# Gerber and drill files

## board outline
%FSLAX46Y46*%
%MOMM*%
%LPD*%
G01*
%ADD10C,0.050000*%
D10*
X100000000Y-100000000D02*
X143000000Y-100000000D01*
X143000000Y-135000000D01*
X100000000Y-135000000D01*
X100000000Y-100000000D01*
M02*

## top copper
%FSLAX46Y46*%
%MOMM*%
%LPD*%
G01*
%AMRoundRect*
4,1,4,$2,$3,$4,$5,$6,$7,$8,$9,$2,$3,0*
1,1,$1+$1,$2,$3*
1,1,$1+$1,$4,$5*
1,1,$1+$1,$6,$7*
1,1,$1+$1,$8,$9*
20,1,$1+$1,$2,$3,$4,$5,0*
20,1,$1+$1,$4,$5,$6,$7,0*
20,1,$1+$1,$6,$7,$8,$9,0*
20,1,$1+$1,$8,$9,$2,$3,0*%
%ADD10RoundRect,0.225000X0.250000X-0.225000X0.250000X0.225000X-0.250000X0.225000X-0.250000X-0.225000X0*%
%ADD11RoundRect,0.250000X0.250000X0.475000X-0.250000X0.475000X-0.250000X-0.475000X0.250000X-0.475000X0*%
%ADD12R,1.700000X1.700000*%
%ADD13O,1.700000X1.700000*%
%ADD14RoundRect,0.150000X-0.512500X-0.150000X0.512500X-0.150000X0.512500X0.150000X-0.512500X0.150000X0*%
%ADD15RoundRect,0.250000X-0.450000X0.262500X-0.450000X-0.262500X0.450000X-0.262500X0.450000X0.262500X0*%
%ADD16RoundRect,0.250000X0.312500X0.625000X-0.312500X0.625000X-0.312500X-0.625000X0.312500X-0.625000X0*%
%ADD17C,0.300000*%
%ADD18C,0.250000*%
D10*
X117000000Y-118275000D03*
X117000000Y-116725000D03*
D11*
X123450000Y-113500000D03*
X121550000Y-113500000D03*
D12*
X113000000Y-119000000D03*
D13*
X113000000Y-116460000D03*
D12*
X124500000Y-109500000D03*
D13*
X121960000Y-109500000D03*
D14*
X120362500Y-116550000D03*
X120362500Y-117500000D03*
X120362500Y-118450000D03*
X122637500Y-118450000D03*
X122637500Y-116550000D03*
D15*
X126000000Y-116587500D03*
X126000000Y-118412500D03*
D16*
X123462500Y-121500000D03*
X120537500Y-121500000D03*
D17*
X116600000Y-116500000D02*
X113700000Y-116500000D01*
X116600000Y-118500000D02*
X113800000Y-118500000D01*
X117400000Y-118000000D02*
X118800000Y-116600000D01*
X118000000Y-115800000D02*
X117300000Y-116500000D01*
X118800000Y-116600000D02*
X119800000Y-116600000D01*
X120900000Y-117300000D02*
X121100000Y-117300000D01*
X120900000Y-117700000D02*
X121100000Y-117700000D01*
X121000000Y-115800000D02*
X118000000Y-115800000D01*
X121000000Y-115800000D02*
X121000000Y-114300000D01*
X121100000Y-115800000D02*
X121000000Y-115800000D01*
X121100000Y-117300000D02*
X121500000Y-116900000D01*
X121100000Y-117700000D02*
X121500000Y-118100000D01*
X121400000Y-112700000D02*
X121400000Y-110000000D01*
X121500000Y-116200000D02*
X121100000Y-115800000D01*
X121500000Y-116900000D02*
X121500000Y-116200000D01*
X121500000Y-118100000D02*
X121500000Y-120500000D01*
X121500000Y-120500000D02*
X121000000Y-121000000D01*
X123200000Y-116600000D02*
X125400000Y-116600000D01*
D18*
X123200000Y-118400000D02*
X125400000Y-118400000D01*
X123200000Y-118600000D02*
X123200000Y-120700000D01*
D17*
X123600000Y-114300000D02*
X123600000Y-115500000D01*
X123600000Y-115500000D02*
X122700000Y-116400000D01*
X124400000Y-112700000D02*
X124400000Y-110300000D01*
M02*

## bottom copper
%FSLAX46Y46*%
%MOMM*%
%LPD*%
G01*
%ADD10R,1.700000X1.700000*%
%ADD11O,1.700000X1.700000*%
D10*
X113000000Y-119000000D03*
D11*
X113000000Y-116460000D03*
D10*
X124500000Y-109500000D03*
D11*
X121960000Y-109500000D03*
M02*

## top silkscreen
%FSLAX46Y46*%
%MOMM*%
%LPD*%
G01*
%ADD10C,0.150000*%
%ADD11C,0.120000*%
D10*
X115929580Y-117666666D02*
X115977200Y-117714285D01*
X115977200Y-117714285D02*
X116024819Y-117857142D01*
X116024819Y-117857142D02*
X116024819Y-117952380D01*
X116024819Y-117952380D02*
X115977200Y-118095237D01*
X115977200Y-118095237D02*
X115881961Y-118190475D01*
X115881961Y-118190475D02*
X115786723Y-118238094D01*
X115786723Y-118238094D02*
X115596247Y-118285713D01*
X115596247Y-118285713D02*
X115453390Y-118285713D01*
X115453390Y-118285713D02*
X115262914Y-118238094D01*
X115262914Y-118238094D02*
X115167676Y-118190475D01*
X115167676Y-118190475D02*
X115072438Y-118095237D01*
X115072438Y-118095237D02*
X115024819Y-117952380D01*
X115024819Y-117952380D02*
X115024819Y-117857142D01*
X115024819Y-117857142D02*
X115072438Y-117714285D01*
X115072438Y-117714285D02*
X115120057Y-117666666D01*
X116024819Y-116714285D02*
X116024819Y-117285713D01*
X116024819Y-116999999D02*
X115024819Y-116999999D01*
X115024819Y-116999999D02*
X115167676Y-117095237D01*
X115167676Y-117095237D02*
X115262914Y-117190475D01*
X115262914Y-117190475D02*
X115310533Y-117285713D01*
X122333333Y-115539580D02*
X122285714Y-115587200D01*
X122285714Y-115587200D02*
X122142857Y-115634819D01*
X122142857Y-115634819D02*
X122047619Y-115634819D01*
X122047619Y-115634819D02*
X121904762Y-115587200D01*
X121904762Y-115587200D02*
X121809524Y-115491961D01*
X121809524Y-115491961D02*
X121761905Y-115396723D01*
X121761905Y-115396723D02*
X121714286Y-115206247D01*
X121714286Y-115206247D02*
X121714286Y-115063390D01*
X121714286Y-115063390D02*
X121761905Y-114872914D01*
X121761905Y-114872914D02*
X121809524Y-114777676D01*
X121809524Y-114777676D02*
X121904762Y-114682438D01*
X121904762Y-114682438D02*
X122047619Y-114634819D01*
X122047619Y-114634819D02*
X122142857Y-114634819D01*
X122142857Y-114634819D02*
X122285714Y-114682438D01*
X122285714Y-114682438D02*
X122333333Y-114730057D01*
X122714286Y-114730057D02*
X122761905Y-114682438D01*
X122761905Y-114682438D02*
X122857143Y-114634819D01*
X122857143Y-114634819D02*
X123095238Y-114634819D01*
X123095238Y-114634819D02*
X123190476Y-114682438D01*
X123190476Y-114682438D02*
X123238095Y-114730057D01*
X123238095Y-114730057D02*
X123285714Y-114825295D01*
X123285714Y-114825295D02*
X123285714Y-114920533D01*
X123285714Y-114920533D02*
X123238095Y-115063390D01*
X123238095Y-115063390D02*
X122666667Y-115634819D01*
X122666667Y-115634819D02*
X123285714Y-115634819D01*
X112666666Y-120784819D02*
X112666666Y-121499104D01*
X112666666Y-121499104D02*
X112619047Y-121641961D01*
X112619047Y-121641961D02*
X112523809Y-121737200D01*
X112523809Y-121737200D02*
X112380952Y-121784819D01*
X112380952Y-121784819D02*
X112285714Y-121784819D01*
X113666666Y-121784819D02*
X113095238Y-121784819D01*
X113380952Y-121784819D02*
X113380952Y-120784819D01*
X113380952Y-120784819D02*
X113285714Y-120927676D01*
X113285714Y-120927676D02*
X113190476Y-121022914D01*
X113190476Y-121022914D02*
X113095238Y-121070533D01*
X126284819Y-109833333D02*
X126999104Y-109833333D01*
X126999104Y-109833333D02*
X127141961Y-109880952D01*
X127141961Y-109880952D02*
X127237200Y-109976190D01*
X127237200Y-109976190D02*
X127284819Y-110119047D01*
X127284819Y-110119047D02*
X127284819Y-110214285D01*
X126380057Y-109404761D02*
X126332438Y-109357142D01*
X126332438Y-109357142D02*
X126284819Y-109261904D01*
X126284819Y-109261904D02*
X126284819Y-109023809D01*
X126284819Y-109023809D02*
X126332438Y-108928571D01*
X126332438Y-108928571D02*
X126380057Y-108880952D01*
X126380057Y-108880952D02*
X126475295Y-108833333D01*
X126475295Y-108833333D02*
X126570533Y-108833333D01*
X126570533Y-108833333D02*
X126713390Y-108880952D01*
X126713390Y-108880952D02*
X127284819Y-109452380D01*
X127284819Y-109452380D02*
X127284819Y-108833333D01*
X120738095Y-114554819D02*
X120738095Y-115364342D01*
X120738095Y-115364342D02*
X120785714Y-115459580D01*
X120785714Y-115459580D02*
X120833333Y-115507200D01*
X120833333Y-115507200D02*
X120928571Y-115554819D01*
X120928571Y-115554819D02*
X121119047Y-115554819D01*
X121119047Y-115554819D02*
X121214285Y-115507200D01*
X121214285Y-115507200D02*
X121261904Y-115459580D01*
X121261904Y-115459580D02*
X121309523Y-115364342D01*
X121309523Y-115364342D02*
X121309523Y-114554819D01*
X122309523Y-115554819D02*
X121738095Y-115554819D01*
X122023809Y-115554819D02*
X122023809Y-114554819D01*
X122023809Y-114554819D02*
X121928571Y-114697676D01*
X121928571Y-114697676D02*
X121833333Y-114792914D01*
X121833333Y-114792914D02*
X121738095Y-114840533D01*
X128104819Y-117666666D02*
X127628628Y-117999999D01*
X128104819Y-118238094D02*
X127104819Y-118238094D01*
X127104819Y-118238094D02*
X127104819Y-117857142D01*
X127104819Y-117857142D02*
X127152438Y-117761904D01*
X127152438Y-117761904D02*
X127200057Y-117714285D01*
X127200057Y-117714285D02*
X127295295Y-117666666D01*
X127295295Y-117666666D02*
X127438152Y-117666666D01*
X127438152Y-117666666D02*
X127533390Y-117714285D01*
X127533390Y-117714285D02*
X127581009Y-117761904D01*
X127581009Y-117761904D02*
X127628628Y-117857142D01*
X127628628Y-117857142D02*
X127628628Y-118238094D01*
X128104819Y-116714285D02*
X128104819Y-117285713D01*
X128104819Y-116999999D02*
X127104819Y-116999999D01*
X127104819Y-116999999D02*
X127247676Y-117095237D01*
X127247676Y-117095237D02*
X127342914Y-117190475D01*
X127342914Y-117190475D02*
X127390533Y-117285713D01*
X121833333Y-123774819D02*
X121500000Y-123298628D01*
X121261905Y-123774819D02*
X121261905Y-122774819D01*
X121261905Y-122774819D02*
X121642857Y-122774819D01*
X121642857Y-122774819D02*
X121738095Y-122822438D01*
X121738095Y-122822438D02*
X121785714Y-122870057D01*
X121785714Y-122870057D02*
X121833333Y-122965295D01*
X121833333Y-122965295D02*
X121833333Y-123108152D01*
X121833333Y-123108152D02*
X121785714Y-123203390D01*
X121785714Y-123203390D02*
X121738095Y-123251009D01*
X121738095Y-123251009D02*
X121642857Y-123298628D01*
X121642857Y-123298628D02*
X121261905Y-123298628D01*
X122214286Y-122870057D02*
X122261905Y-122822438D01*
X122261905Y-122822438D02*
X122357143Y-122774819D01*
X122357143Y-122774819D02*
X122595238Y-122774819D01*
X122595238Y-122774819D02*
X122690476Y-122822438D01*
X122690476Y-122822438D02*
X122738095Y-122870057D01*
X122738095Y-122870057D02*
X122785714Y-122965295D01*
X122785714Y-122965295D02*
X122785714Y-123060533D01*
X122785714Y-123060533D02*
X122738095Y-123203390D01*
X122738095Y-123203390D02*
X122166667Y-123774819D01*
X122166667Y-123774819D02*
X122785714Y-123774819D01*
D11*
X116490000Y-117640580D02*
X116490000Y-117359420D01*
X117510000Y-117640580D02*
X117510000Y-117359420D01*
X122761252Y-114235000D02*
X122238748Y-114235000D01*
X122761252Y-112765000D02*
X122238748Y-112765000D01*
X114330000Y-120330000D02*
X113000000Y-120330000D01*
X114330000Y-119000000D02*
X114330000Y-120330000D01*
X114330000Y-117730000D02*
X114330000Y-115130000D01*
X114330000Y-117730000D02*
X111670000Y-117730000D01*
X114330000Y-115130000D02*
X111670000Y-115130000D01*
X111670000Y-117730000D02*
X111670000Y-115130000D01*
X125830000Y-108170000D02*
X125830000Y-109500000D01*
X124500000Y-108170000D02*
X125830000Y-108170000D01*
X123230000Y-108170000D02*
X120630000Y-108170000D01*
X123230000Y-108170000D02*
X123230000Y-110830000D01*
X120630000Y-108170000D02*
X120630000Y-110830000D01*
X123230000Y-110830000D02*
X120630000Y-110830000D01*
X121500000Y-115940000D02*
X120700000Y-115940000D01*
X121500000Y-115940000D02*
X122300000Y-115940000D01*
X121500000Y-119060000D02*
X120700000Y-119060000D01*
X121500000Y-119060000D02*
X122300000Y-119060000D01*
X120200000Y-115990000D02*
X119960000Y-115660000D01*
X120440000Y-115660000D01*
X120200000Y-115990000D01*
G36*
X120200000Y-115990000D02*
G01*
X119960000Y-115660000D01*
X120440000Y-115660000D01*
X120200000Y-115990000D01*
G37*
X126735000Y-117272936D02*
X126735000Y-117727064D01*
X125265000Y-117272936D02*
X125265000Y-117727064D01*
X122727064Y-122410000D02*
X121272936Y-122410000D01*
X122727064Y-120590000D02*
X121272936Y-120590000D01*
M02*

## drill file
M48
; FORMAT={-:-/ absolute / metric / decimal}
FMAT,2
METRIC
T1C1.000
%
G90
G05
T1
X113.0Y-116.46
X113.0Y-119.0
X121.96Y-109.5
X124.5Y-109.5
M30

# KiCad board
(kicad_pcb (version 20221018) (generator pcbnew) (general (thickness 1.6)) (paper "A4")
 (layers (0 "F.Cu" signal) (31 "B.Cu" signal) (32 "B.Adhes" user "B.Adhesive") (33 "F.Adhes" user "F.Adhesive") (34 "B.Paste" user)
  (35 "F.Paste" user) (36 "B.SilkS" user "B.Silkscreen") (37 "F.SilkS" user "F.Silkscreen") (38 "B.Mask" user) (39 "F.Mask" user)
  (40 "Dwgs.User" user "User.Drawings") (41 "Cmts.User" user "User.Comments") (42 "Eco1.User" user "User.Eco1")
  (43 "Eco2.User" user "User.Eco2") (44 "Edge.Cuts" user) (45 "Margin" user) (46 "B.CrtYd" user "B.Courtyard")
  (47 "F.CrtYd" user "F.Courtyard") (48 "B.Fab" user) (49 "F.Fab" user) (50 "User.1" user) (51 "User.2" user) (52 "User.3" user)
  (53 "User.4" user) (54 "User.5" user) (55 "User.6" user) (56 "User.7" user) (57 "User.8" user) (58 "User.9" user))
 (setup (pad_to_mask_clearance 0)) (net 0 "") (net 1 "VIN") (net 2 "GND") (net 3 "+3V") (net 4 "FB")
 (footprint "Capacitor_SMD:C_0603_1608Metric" (layer "F.Cu") (at 117 117.5 90)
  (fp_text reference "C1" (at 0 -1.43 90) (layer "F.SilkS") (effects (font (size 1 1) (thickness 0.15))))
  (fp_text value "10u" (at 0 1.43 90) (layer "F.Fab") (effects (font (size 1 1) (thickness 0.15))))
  (fp_line (start -0.14058 -0.51) (end 0.14058 -0.51) (stroke (width 0.12) (type solid)) (layer "F.SilkS"))
  (fp_line (start -0.14058 0.51) (end 0.14058 0.51) (stroke (width 0.12) (type solid)) (layer "F.SilkS"))
  (pad "1" smd roundrect (at -0.775 0 90) (size 0.9 0.95) (layers "F.Cu" "F.Paste" "F.Mask") (roundrect_rratio 0.25) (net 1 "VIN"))
  (pad "2" smd roundrect (at 0.775 0 90) (size 0.9 0.95) (layers "F.Cu" "F.Paste" "F.Mask") (roundrect_rratio 0.25) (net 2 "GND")))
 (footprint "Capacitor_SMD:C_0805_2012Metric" (layer "F.Cu") (at 122.5 113.5 180)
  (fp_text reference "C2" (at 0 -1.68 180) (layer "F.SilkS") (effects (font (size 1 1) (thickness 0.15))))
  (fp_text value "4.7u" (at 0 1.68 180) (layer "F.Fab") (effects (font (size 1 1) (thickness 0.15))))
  (fp_line (start -0.261252 -0.735) (end 0.261252 -0.735) (stroke (width 0.12) (type solid)) (layer "F.SilkS"))
  (fp_line (start -0.261252 0.735) (end 0.261252 0.735) (stroke (width 0.12) (type solid)) (layer "F.SilkS"))
  (pad "1" smd roundrect (at -0.95 0 180) (size 1 1.45) (layers "F.Cu" "F.Paste" "F.Mask") (roundrect_rratio 0.25) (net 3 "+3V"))
  (pad "2" smd roundrect (at 0.95 0 180) (size 1 1.45) (layers "F.Cu" "F.Paste" "F.Mask") (roundrect_rratio 0.25) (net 2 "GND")))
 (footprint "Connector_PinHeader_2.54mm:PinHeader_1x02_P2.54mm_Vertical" (layer "F.Cu") (at 113 119 180)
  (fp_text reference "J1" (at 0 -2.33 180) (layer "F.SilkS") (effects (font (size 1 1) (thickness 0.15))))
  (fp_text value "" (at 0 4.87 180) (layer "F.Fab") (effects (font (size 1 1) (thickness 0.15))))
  (fp_line (start -1.33 -1.33) (end 0 -1.33) (stroke (width 0.12) (type solid)) (layer "F.SilkS"))
  (fp_line (start -1.33 0) (end -1.33 -1.33) (stroke (width 0.12) (type solid)) (layer "F.SilkS"))
  (fp_line (start -1.33 1.27) (end -1.33 3.87) (stroke (width 0.12) (type solid)) (layer "F.SilkS"))
  (fp_line (start -1.33 1.27) (end 1.33 1.27) (stroke (width 0.12) (type solid)) (layer "F.SilkS"))
  (fp_line (start -1.33 3.87) (end 1.33 3.87) (stroke (width 0.12) (type solid)) (layer "F.SilkS"))
  (fp_line (start 1.33 1.27) (end 1.33 3.87) (stroke (width 0.12) (type solid)) (layer "F.SilkS"))
  (pad "1" thru_hole rect (at 0 0 180) (size 1.7 1.7) (drill 1) (layers "*.Cu" "*.Mask") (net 1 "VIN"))
  (pad "2" thru_hole oval (at 0 2.54 180) (size 1.7 1.7) (drill 1) (layers "*.Cu" "*.Mask") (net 2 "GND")))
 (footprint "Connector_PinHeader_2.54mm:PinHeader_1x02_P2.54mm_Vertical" (layer "F.Cu") (at 124.5 109.5 -90)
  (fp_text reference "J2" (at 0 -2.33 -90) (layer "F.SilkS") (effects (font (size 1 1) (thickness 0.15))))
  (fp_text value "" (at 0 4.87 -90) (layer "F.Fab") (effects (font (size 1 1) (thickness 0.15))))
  (fp_line (start -1.33 -1.33) (end 0 -1.33) (stroke (width 0.12) (type solid)) (layer "F.SilkS"))
  (fp_line (start -1.33 0) (end -1.33 -1.33) (stroke (width 0.12) (type solid)) (layer "F.SilkS"))
  (fp_line (start -1.33 1.27) (end -1.33 3.87) (stroke (width 0.12) (type solid)) (layer "F.SilkS"))
  (fp_line (start -1.33 1.27) (end 1.33 1.27) (stroke (width 0.12) (type solid)) (layer "F.SilkS"))
  (fp_line (start -1.33 3.87) (end 1.33 3.87) (stroke (width 0.12) (type solid)) (layer "F.SilkS"))
  (fp_line (start 1.33 1.27) (end 1.33 3.87) (stroke (width 0.12) (type solid)) (layer "F.SilkS"))
  (pad "1" thru_hole rect (at 0 0 270) (size 1.7 1.7) (drill 1) (layers "*.Cu" "*.Mask") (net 3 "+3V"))
  (pad "2" thru_hole oval (at 0 2.54 270) (size 1.7 1.7) (drill 1) (layers "*.Cu" "*.Mask") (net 2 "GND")))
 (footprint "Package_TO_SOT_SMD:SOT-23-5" (layer "F.Cu") (at 121.5 117.5)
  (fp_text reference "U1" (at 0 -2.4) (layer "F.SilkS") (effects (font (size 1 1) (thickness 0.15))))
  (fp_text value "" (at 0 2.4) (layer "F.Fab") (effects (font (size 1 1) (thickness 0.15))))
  (fp_line (start 0 -1.56) (end -0.8 -1.56) (stroke (width 0.12) (type solid)) (layer "F.SilkS"))
  (fp_line (start 0 -1.56) (end 0.8 -1.56) (stroke (width 0.12) (type solid)) (layer "F.SilkS"))
  (fp_line (start 0 1.56) (end -0.8 1.56) (stroke (width 0.12) (type solid)) (layer "F.SilkS"))
  (fp_line (start 0 1.56) (end 0.8 1.56) (stroke (width 0.12) (type solid)) (layer "F.SilkS"))
  (fp_poly
   (pts (xy -1.3 -1.51) (xy -1.54 -1.84) (xy -1.06 -1.84) (xy -1.3 -1.51)) (stroke (width 0.12) (type solid)) (fill solid) (layer "F.SilkS"))
  (pad "1" smd roundrect (at -1.1375 -0.95) (size 1.325 0.6) (layers "F.Cu" "F.Paste" "F.Mask") (roundrect_rratio 0.25) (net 1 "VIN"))
  (pad "2" smd roundrect (at -1.1375 0) (size 1.325 0.6) (layers "F.Cu" "F.Paste" "F.Mask") (roundrect_rratio 0.25) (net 2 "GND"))
  (pad "3" smd roundrect (at -1.1375 0.95) (size 1.325 0.6) (layers "F.Cu" "F.Paste" "F.Mask") (roundrect_rratio 0.25))
  (pad "4" smd roundrect (at 1.1375 0.95) (size 1.325 0.6) (layers "F.Cu" "F.Paste" "F.Mask") (roundrect_rratio 0.25) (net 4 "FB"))
  (pad "5" smd roundrect (at 1.1375 -0.95) (size 1.325 0.6) (layers "F.Cu" "F.Paste" "F.Mask") (roundrect_rratio 0.25) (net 3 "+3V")))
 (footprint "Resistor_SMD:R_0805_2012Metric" (layer "F.Cu") (at 126 117.5 -90)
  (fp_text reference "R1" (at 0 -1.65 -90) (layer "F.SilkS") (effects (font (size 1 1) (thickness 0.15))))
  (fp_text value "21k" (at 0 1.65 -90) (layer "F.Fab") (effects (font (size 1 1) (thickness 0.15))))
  (fp_line (start -0.227064 -0.735) (end 0.227064 -0.735) (stroke (width 0.12) (type solid)) (layer "F.SilkS"))
  (fp_line (start -0.227064 0.735) (end 0.227064 0.735) (stroke (width 0.12) (type solid)) (layer "F.SilkS"))
  (pad "1" smd roundrect (at -0.9125 0 270) (size 1.025 1.4) (layers "F.Cu" "F.Paste" "F.Mask") (roundrect_rratio 0.243902) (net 3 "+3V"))
  (pad "2" smd roundrect (at 0.9125 0 270) (size 1.025 1.4) (layers "F.Cu" "F.Paste" "F.Mask") (roundrect_rratio 0.243902) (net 4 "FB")))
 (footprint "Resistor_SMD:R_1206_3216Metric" (layer "F.Cu") (at 122 121.5 180)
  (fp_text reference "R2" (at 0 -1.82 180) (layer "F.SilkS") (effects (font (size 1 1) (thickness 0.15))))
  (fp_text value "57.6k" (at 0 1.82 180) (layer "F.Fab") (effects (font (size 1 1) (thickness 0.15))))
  (fp_line (start -0.727064 -0.91) (end 0.727064 -0.91) (stroke (width 0.12) (type solid)) (layer "F.SilkS"))
  (fp_line (start -0.727064 0.91) (end 0.727064 0.91) (stroke (width 0.12) (type solid)) (layer "F.SilkS"))
  (pad "1" smd roundrect (at -1.4625 0 180) (size 1.125 1.75) (layers "F.Cu" "F.Paste" "F.Mask") (roundrect_rratio 0.222222) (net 4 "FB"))
  (pad "2" smd roundrect (at 1.4625 0 180) (size 1.125 1.75) (layers "F.Cu" "F.Paste" "F.Mask") (roundrect_rratio 0.222222) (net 2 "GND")))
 (gr_rect (start 100 100) (end 143 135) (stroke (width 0.05) (type default)) (fill none) (layer "Edge.Cuts"))
 (segment (start 116.6 116.5) (end 113.7 116.5) (width 0.3) (layer "F.Cu") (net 2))
 (segment (start 116.6 118.5) (end 113.8 118.5) (width 0.3) (layer "F.Cu") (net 1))
 (segment (start 117.4 118) (end 118.8 116.6) (width 0.3) (layer "F.Cu") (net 1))
 (segment (start 118 115.8) (end 117.3 116.5) (width 0.3) (layer "F.Cu") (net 2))
 (segment (start 118.8 116.6) (end 119.8 116.6) (width 0.3) (layer "F.Cu") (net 1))
 (segment (start 120.9 117.3) (end 121.1 117.3) (width 0.3) (layer "F.Cu") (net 2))
 (segment (start 120.9 117.7) (end 121.1 117.7) (width 0.3) (layer "F.Cu") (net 2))
 (segment (start 121 115.8) (end 118 115.8) (width 0.3) (layer "F.Cu") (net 2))
 (segment (start 121 115.8) (end 121 114.3) (width 0.3) (layer "F.Cu") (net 2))
 (segment (start 121.1 115.8) (end 121 115.8) (width 0.3) (layer "F.Cu") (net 2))
 (segment (start 121.1 117.3) (end 121.5 116.9) (width 0.3) (layer "F.Cu") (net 2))
 (segment (start 121.1 117.7) (end 121.5 118.1) (width 0.3) (layer "F.Cu") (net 2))
 (segment (start 121.4 112.7) (end 121.4 110) (width 0.3) (layer "F.Cu") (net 2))
 (segment (start 121.5 116.2) (end 121.1 115.8) (width 0.3) (layer "F.Cu") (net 2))
 (segment (start 121.5 116.9) (end 121.5 116.2) (width 0.3) (layer "F.Cu") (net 2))
 (segment (start 121.5 118.1) (end 121.5 120.5) (width 0.3) (layer "F.Cu") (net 2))
 (segment (start 121.5 120.5) (end 121 121) (width 0.3) (layer "F.Cu") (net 2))
 (segment (start 123.2 116.6) (end 125.4 116.6) (width 0.3) (layer "F.Cu") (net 3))
 (segment (start 123.2 118.4) (end 125.4 118.4) (width 0.25) (layer "F.Cu") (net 4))
 (segment (start 123.2 118.6) (end 123.2 120.7) (width 0.25) (layer "F.Cu") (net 4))
 (segment (start 123.6 114.3) (end 123.6 115.5) (width 0.3) (layer "F.Cu") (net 3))
 (segment (start 123.6 115.5) (end 122.7 116.4) (width 0.3) (layer "F.Cu") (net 3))
 (segment (start 124.4 112.7) (end 124.4 110.3) (width 0.3) (layer "F.Cu") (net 3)))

